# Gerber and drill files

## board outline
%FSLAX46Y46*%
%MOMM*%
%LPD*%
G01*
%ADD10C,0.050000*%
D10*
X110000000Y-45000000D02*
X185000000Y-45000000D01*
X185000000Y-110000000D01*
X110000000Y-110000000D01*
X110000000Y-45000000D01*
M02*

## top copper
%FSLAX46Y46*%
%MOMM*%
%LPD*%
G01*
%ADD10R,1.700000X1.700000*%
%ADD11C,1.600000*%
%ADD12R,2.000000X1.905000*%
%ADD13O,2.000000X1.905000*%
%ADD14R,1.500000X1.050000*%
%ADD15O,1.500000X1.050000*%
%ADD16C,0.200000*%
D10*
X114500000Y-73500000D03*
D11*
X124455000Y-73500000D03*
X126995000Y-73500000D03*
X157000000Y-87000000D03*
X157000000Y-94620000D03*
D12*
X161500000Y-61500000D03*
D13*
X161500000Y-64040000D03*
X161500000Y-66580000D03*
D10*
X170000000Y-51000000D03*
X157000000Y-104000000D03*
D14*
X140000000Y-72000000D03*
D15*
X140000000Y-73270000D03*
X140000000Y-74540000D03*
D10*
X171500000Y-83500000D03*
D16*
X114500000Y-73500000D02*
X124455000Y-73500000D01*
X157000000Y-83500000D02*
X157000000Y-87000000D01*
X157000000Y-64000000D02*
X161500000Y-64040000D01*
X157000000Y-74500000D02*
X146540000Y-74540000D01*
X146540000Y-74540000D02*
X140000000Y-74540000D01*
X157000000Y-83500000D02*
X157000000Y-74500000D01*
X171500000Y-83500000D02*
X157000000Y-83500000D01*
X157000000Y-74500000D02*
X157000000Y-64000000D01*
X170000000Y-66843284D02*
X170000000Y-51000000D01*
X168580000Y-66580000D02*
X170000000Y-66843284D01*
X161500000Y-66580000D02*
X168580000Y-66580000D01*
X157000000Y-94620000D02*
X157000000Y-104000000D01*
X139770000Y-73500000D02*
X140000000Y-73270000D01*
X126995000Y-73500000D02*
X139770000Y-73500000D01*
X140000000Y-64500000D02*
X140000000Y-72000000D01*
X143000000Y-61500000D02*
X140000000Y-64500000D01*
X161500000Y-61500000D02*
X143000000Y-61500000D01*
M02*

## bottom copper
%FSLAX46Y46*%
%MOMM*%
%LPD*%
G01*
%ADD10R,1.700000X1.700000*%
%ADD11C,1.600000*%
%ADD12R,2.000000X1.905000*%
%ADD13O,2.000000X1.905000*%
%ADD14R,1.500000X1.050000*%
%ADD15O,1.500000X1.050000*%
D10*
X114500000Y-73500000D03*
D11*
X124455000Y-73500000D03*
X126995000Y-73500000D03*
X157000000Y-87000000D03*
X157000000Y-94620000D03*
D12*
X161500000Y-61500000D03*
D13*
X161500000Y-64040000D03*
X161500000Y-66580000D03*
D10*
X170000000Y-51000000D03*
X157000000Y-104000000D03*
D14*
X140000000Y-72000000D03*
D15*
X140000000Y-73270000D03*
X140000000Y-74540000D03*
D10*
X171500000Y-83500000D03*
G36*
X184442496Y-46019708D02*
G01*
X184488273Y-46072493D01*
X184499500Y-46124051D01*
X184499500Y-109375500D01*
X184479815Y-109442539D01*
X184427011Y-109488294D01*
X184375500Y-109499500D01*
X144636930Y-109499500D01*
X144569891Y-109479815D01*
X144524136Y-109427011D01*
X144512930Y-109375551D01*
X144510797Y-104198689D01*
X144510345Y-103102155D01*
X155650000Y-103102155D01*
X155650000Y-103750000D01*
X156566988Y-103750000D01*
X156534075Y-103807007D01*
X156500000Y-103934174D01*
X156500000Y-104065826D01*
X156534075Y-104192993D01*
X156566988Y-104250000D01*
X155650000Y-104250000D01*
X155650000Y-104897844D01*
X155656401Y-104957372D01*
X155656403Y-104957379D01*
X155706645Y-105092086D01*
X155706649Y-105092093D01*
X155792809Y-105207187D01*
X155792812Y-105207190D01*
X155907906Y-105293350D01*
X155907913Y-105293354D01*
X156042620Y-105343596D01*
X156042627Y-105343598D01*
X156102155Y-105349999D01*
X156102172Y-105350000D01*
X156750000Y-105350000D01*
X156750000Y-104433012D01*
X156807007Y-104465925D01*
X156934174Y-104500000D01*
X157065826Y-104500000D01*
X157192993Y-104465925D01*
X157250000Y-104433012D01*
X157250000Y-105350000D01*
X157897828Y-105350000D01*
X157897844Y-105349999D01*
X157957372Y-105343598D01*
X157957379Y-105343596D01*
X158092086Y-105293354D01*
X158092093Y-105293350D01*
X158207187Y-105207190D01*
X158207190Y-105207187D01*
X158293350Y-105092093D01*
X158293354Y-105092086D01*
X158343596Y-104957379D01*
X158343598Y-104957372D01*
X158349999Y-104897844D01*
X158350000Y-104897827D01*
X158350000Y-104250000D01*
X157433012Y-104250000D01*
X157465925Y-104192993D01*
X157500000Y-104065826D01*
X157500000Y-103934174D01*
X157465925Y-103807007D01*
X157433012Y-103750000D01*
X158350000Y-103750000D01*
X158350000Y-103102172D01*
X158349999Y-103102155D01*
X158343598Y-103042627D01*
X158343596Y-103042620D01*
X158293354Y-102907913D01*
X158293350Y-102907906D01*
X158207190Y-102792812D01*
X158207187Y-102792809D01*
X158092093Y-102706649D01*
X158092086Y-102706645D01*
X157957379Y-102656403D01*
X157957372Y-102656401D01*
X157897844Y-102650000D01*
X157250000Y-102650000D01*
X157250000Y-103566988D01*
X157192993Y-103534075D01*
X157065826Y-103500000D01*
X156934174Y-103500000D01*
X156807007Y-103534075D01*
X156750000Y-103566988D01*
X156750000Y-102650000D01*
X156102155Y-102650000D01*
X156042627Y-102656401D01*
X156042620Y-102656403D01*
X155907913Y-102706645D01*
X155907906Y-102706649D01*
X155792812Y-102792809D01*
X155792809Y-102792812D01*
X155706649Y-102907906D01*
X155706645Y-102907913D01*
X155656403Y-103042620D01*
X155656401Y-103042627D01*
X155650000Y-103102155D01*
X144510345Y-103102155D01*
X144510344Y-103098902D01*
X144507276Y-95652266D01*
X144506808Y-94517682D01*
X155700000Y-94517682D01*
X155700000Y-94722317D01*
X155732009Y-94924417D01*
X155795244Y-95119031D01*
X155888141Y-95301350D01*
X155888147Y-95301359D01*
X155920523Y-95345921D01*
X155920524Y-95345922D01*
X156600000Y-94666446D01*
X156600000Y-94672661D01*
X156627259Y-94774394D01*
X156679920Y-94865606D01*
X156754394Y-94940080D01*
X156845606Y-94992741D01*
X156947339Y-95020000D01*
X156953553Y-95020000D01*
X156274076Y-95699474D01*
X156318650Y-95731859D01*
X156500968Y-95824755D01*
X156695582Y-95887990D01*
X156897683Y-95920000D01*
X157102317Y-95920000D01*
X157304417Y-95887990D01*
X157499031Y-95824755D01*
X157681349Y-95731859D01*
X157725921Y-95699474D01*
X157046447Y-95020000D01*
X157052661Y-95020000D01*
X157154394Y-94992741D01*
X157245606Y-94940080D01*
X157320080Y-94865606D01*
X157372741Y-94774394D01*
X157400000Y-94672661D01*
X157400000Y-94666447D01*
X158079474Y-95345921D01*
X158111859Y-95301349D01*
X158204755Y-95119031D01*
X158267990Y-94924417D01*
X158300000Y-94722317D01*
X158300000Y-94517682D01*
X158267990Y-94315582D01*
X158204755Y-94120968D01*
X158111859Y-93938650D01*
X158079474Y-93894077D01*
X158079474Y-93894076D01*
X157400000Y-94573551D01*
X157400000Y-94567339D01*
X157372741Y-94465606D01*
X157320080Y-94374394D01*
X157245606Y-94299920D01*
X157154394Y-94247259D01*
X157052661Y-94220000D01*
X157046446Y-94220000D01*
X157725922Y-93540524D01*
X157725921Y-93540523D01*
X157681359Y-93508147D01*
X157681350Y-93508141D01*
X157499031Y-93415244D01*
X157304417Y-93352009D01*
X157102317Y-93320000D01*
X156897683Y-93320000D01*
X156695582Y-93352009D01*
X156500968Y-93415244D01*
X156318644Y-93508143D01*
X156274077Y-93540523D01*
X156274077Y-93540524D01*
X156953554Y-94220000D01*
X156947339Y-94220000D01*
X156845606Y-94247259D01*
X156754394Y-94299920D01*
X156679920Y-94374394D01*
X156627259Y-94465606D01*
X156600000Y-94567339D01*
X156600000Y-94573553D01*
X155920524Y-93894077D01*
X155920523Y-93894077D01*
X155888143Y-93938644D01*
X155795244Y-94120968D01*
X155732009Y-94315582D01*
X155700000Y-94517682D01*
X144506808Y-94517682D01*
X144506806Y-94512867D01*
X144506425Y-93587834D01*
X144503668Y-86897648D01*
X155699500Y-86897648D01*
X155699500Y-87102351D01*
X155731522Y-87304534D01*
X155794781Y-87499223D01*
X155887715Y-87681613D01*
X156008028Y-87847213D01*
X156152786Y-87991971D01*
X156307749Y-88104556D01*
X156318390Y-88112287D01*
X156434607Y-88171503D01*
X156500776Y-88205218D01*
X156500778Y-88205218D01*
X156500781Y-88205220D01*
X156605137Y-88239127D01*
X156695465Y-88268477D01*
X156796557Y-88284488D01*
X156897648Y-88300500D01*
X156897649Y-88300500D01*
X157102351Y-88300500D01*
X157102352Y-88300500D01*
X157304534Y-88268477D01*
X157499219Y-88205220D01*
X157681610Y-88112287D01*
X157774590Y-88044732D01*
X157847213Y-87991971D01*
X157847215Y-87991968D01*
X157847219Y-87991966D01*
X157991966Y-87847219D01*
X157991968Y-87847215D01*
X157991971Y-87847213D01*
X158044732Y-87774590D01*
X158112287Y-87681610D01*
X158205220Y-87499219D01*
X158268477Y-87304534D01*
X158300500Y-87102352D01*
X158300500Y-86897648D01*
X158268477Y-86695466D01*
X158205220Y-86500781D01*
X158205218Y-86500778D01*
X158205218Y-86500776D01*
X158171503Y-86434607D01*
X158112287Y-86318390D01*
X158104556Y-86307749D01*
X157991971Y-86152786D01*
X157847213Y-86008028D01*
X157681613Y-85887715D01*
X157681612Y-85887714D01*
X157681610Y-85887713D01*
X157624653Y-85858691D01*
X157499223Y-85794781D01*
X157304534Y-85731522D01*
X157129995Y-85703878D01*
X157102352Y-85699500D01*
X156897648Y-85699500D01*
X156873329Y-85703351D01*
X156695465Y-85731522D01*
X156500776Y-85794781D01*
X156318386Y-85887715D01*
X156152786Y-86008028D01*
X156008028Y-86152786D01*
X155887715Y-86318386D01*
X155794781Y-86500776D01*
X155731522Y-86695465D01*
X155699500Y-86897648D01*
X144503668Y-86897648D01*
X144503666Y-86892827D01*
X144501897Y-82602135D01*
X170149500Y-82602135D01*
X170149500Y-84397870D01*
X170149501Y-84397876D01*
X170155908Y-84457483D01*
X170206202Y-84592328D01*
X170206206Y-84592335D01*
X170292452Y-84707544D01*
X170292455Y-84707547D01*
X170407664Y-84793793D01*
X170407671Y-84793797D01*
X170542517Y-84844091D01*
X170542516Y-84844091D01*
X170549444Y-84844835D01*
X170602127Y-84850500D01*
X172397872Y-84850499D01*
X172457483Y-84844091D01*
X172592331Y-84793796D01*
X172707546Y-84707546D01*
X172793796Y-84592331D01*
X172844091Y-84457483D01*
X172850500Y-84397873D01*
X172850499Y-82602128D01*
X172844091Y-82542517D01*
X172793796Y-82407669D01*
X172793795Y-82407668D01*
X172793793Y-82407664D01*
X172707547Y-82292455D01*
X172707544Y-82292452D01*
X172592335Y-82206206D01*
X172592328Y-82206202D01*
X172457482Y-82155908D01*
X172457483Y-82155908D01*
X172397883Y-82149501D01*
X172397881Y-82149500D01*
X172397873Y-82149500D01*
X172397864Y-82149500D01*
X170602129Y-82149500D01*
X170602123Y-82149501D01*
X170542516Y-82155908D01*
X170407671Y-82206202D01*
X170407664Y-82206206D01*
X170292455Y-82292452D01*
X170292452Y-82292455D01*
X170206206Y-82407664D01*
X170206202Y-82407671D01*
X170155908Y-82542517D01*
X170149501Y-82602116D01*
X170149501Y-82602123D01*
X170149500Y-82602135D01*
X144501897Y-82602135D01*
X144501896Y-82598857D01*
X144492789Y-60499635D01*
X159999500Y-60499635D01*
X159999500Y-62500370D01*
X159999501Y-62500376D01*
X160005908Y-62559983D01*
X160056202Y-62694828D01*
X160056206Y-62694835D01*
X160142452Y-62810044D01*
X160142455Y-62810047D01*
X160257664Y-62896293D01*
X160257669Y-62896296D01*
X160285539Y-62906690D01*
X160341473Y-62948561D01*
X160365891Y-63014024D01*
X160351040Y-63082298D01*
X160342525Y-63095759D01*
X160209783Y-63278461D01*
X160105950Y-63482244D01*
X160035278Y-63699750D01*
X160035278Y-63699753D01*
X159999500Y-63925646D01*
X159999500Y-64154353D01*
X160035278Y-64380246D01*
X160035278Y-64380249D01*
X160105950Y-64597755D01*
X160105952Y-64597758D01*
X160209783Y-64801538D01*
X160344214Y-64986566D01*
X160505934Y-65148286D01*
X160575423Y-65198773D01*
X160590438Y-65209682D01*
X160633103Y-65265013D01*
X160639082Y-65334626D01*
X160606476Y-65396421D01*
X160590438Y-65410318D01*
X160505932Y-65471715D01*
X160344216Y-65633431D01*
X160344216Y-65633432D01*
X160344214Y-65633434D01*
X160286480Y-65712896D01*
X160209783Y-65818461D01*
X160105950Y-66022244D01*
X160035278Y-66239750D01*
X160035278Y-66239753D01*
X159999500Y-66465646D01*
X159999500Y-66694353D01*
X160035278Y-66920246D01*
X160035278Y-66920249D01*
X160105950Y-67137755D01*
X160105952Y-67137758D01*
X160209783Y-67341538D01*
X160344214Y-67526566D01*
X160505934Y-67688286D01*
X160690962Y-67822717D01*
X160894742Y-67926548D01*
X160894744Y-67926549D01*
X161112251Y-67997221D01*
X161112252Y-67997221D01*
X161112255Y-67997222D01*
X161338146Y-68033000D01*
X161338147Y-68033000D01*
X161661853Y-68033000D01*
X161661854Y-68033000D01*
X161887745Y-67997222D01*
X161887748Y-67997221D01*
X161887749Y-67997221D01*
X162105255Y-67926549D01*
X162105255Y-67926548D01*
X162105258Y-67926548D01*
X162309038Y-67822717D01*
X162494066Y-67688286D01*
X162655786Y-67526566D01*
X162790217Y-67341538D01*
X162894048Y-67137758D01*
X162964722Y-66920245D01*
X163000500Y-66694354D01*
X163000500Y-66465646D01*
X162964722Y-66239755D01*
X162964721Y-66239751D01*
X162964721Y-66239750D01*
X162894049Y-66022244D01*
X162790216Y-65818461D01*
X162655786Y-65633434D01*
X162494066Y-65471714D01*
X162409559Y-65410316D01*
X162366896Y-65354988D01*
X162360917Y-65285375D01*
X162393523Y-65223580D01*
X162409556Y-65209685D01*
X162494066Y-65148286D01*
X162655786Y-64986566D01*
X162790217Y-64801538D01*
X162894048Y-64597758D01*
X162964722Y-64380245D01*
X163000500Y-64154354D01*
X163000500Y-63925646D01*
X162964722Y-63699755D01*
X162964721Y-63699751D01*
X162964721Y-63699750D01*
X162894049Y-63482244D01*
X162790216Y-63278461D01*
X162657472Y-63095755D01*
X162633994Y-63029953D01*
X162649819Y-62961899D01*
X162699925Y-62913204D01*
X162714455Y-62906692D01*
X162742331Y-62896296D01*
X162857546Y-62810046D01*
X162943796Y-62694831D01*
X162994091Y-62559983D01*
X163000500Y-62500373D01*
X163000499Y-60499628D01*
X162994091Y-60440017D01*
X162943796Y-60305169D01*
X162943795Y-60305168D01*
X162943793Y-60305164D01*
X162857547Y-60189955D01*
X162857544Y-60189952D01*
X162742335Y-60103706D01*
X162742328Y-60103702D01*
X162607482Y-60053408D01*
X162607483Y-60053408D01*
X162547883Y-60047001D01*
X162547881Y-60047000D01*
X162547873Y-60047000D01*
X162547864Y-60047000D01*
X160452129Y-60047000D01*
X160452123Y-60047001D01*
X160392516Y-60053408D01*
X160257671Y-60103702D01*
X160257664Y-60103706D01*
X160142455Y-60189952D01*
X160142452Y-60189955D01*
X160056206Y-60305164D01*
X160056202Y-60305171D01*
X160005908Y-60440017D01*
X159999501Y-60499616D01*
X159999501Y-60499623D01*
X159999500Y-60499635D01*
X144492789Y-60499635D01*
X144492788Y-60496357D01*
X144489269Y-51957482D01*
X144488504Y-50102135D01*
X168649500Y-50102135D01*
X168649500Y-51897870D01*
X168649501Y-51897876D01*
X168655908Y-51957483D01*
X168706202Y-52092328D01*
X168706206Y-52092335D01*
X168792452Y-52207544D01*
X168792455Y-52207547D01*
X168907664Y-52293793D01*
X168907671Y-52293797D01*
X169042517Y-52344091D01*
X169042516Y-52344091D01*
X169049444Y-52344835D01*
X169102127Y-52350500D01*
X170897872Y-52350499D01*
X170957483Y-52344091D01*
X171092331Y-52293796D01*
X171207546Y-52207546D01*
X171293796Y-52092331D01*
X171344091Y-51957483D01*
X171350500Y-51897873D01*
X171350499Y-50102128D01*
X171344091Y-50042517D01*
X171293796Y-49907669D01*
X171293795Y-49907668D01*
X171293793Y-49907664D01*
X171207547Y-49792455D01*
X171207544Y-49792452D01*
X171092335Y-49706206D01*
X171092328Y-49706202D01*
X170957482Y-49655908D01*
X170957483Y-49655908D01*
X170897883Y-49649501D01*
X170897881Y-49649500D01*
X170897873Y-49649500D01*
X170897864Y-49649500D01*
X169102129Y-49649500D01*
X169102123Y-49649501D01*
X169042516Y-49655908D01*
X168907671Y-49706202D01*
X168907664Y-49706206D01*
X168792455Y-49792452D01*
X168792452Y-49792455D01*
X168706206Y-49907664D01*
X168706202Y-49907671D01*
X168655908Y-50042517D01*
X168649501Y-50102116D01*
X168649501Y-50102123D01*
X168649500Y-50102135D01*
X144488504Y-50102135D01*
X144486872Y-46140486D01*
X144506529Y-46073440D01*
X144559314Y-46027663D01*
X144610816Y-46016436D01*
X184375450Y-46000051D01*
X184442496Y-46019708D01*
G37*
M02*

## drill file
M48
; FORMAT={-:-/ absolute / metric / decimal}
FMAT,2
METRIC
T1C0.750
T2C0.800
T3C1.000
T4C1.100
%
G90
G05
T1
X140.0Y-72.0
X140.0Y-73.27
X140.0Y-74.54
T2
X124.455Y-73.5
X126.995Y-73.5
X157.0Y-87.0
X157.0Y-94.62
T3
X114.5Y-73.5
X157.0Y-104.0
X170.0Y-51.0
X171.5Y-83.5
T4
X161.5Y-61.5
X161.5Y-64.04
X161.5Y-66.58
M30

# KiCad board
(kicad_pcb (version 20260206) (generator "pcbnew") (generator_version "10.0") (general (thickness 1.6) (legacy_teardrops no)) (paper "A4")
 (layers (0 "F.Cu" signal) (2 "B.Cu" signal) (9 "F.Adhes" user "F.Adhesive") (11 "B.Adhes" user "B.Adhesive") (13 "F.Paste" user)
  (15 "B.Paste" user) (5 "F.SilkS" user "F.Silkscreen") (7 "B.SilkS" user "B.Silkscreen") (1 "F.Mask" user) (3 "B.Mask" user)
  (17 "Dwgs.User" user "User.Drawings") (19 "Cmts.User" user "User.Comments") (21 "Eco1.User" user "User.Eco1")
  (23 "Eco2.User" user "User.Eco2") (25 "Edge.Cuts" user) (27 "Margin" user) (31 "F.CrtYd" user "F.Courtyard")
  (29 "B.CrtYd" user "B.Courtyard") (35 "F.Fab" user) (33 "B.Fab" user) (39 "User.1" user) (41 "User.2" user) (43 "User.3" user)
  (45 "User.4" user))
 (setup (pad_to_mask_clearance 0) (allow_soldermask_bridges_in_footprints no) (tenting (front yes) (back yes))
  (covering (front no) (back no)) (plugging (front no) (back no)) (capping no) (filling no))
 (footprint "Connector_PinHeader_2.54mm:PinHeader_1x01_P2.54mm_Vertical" (layer "F.Cu") (at 114.5 73.5)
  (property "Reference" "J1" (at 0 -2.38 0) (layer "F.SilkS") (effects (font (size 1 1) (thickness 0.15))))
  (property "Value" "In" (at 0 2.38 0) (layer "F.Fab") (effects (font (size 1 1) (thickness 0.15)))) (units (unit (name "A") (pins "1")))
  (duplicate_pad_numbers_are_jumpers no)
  (pad "1" thru_hole rect (at 0 0) (size 1.7 1.7) (drill 1) (layers "*.Cu" "*.Mask") (remove_unused_layers no) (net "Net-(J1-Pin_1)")))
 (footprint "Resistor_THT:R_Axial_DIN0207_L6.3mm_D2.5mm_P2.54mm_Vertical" (layer "F.Cu") (at 124.455 73.5)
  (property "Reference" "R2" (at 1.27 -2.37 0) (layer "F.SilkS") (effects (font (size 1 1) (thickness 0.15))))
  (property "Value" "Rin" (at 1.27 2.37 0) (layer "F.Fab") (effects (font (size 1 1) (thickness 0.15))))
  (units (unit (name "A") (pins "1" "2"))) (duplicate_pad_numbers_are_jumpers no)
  (pad "1" thru_hole circle (at 0 0) (size 1.6 1.6) (drill 0.8) (layers "*.Cu" "*.Mask") (remove_unused_layers no) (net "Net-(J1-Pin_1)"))
  (pad "2" thru_hole circle (at 2.54 0) (size 1.6 1.6) (drill 0.8) (layers "*.Cu" "*.Mask") (remove_unused_layers no) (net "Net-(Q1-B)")))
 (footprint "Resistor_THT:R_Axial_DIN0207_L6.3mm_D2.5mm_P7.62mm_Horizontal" (layer "F.Cu") (at 157 87 -90)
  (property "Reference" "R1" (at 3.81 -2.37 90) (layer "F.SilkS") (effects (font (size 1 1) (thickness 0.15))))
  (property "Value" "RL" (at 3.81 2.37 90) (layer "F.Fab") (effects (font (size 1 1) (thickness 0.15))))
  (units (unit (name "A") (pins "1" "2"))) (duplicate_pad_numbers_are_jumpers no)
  (pad "1" thru_hole circle (at 0 0 270) (size 1.6 1.6) (drill 0.8) (layers "*.Cu" "*.Mask") (remove_unused_layers no)
   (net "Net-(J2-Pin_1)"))
  (pad "2" thru_hole circle (at 7.62 0 270) (size 1.6 1.6) (drill 0.8) (layers "*.Cu" "*.Mask") (remove_unused_layers no) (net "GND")))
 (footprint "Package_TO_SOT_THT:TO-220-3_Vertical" (layer "F.Cu") (at 161.5 61.5 -90)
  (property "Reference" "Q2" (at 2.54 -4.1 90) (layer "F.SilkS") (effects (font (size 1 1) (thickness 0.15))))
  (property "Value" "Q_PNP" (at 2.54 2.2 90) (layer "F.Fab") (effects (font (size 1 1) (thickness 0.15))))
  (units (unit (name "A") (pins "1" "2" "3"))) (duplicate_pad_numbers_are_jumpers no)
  (pad "1" thru_hole rect (at 0 0 270) (size 1.905 2) (drill 1.1) (layers "*.Cu" "*.Mask") (remove_unused_layers no) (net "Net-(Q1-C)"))
  (pad "2" thru_hole oval (at 2.54 0 270) (size 1.905 2) (drill 1.1) (layers "*.Cu" "*.Mask") (remove_unused_layers no)
   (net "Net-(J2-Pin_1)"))
  (pad "3" thru_hole oval (at 5.08 0 270) (size 1.905 2) (drill 1.1) (layers "*.Cu" "*.Mask") (remove_unused_layers no) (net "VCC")))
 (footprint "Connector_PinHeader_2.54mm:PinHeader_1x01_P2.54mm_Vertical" (layer "F.Cu") (at 170 51)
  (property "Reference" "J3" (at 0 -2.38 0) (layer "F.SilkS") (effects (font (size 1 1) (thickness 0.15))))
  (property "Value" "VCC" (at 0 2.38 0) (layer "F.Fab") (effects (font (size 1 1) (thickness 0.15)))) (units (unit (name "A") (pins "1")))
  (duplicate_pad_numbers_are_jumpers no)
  (pad "1" thru_hole rect (at 0 0) (size 1.7 1.7) (drill 1) (layers "*.Cu" "*.Mask") (remove_unused_layers no) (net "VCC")))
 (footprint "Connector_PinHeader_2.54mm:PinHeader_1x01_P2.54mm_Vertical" (layer "F.Cu") (at 157 104)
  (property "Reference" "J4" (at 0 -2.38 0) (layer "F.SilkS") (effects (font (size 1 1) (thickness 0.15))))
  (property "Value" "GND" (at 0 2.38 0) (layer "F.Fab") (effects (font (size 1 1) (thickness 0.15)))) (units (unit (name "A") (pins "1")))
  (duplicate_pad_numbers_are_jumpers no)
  (pad "1" thru_hole rect (at 0 0) (size 1.7 1.7) (drill 1) (layers "*.Cu" "*.Mask") (remove_unused_layers no) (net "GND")))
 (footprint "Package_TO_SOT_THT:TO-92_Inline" (layer "F.Cu") (at 140 72 -90)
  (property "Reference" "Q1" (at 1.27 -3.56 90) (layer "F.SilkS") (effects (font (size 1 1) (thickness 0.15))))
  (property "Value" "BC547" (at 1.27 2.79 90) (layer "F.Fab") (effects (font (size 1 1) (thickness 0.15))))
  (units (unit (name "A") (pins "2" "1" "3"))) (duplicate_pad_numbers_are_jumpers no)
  (pad "1" thru_hole rect (at 0 0 270) (size 1.05 1.5) (drill 0.75) (layers "*.Cu" "*.Mask") (remove_unused_layers no) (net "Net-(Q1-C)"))
  (pad "2" thru_hole oval (at 1.27 0 270) (size 1.05 1.5) (drill 0.75) (layers "*.Cu" "*.Mask") (remove_unused_layers no) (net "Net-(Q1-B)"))
  (pad "3" thru_hole oval (at 2.54 0 270) (size 1.05 1.5) (drill 0.75) (layers "*.Cu" "*.Mask") (remove_unused_layers no)
   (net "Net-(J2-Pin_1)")))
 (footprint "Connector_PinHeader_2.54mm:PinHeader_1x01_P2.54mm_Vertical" (layer "F.Cu") (at 171.5 83.5)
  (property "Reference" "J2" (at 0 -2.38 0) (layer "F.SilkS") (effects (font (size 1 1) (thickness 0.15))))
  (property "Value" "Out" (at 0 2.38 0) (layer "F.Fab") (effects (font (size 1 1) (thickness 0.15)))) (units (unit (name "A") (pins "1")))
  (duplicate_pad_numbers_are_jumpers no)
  (pad "1" thru_hole rect (at 0 0) (size 1.7 1.7) (drill 1) (layers "*.Cu" "*.Mask") (remove_unused_layers no) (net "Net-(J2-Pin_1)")))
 (gr_rect (start 110 45) (end 185 110) (stroke (width 0.05) (type default)) (fill no) (layer "Edge.Cuts"))
 (segment (start 114.5 73.5) (end 124.455 73.5) (width 0.2) (layer "F.Cu") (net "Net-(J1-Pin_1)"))
 (segment (start 157 83.5) (end 157 87) (width 0.2) (layer "F.Cu") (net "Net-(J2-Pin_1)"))
 (segment (start 157 64) (end 161.5 64.04) (width 0.2) (layer "F.Cu") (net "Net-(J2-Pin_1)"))
 (segment (start 157 74.5) (end 146.54 74.54) (width 0.2) (layer "F.Cu") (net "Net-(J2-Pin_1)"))
 (segment (start 146.54 74.54) (end 140 74.54) (width 0.2) (layer "F.Cu") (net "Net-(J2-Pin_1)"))
 (segment (start 157 83.5) (end 157 74.5) (width 0.2) (layer "F.Cu") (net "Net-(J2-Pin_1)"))
 (segment (start 171.5 83.5) (end 157 83.5) (width 0.2) (layer "F.Cu") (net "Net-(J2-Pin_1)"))
 (segment (start 157 74.5) (end 157 64) (width 0.2) (layer "F.Cu") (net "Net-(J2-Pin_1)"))
 (segment (start 170 66.843284) (end 170 51) (width 0.2) (layer "F.Cu") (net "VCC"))
 (segment (start 168.58 66.58) (end 170 66.843284) (width 0.2) (layer "F.Cu") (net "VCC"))
 (segment (start 161.5 66.58) (end 168.58 66.58) (width 0.2) (layer "F.Cu") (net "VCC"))
 (segment (start 157 94.62) (end 157 104) (width 0.2) (layer "F.Cu") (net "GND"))
 (segment (start 139.77 73.5) (end 140 73.27) (width 0.2) (layer "F.Cu") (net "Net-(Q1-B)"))
 (segment (start 126.995 73.5) (end 139.77 73.5) (width 0.2) (layer "F.Cu") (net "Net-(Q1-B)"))
 (segment (start 140 64.5) (end 140 72) (width 0.2) (layer "F.Cu") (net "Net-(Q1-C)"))
 (segment (start 143 61.5) (end 140 64.5) (width 0.2) (layer "F.Cu") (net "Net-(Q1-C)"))
 (segment (start 161.5 61.5) (end 143 61.5) (width 0.2) (layer "F.Cu") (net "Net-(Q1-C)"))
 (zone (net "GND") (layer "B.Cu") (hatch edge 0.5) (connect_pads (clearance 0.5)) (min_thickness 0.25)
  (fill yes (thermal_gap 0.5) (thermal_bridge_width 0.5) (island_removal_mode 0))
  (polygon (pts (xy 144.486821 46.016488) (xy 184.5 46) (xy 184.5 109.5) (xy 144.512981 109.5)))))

